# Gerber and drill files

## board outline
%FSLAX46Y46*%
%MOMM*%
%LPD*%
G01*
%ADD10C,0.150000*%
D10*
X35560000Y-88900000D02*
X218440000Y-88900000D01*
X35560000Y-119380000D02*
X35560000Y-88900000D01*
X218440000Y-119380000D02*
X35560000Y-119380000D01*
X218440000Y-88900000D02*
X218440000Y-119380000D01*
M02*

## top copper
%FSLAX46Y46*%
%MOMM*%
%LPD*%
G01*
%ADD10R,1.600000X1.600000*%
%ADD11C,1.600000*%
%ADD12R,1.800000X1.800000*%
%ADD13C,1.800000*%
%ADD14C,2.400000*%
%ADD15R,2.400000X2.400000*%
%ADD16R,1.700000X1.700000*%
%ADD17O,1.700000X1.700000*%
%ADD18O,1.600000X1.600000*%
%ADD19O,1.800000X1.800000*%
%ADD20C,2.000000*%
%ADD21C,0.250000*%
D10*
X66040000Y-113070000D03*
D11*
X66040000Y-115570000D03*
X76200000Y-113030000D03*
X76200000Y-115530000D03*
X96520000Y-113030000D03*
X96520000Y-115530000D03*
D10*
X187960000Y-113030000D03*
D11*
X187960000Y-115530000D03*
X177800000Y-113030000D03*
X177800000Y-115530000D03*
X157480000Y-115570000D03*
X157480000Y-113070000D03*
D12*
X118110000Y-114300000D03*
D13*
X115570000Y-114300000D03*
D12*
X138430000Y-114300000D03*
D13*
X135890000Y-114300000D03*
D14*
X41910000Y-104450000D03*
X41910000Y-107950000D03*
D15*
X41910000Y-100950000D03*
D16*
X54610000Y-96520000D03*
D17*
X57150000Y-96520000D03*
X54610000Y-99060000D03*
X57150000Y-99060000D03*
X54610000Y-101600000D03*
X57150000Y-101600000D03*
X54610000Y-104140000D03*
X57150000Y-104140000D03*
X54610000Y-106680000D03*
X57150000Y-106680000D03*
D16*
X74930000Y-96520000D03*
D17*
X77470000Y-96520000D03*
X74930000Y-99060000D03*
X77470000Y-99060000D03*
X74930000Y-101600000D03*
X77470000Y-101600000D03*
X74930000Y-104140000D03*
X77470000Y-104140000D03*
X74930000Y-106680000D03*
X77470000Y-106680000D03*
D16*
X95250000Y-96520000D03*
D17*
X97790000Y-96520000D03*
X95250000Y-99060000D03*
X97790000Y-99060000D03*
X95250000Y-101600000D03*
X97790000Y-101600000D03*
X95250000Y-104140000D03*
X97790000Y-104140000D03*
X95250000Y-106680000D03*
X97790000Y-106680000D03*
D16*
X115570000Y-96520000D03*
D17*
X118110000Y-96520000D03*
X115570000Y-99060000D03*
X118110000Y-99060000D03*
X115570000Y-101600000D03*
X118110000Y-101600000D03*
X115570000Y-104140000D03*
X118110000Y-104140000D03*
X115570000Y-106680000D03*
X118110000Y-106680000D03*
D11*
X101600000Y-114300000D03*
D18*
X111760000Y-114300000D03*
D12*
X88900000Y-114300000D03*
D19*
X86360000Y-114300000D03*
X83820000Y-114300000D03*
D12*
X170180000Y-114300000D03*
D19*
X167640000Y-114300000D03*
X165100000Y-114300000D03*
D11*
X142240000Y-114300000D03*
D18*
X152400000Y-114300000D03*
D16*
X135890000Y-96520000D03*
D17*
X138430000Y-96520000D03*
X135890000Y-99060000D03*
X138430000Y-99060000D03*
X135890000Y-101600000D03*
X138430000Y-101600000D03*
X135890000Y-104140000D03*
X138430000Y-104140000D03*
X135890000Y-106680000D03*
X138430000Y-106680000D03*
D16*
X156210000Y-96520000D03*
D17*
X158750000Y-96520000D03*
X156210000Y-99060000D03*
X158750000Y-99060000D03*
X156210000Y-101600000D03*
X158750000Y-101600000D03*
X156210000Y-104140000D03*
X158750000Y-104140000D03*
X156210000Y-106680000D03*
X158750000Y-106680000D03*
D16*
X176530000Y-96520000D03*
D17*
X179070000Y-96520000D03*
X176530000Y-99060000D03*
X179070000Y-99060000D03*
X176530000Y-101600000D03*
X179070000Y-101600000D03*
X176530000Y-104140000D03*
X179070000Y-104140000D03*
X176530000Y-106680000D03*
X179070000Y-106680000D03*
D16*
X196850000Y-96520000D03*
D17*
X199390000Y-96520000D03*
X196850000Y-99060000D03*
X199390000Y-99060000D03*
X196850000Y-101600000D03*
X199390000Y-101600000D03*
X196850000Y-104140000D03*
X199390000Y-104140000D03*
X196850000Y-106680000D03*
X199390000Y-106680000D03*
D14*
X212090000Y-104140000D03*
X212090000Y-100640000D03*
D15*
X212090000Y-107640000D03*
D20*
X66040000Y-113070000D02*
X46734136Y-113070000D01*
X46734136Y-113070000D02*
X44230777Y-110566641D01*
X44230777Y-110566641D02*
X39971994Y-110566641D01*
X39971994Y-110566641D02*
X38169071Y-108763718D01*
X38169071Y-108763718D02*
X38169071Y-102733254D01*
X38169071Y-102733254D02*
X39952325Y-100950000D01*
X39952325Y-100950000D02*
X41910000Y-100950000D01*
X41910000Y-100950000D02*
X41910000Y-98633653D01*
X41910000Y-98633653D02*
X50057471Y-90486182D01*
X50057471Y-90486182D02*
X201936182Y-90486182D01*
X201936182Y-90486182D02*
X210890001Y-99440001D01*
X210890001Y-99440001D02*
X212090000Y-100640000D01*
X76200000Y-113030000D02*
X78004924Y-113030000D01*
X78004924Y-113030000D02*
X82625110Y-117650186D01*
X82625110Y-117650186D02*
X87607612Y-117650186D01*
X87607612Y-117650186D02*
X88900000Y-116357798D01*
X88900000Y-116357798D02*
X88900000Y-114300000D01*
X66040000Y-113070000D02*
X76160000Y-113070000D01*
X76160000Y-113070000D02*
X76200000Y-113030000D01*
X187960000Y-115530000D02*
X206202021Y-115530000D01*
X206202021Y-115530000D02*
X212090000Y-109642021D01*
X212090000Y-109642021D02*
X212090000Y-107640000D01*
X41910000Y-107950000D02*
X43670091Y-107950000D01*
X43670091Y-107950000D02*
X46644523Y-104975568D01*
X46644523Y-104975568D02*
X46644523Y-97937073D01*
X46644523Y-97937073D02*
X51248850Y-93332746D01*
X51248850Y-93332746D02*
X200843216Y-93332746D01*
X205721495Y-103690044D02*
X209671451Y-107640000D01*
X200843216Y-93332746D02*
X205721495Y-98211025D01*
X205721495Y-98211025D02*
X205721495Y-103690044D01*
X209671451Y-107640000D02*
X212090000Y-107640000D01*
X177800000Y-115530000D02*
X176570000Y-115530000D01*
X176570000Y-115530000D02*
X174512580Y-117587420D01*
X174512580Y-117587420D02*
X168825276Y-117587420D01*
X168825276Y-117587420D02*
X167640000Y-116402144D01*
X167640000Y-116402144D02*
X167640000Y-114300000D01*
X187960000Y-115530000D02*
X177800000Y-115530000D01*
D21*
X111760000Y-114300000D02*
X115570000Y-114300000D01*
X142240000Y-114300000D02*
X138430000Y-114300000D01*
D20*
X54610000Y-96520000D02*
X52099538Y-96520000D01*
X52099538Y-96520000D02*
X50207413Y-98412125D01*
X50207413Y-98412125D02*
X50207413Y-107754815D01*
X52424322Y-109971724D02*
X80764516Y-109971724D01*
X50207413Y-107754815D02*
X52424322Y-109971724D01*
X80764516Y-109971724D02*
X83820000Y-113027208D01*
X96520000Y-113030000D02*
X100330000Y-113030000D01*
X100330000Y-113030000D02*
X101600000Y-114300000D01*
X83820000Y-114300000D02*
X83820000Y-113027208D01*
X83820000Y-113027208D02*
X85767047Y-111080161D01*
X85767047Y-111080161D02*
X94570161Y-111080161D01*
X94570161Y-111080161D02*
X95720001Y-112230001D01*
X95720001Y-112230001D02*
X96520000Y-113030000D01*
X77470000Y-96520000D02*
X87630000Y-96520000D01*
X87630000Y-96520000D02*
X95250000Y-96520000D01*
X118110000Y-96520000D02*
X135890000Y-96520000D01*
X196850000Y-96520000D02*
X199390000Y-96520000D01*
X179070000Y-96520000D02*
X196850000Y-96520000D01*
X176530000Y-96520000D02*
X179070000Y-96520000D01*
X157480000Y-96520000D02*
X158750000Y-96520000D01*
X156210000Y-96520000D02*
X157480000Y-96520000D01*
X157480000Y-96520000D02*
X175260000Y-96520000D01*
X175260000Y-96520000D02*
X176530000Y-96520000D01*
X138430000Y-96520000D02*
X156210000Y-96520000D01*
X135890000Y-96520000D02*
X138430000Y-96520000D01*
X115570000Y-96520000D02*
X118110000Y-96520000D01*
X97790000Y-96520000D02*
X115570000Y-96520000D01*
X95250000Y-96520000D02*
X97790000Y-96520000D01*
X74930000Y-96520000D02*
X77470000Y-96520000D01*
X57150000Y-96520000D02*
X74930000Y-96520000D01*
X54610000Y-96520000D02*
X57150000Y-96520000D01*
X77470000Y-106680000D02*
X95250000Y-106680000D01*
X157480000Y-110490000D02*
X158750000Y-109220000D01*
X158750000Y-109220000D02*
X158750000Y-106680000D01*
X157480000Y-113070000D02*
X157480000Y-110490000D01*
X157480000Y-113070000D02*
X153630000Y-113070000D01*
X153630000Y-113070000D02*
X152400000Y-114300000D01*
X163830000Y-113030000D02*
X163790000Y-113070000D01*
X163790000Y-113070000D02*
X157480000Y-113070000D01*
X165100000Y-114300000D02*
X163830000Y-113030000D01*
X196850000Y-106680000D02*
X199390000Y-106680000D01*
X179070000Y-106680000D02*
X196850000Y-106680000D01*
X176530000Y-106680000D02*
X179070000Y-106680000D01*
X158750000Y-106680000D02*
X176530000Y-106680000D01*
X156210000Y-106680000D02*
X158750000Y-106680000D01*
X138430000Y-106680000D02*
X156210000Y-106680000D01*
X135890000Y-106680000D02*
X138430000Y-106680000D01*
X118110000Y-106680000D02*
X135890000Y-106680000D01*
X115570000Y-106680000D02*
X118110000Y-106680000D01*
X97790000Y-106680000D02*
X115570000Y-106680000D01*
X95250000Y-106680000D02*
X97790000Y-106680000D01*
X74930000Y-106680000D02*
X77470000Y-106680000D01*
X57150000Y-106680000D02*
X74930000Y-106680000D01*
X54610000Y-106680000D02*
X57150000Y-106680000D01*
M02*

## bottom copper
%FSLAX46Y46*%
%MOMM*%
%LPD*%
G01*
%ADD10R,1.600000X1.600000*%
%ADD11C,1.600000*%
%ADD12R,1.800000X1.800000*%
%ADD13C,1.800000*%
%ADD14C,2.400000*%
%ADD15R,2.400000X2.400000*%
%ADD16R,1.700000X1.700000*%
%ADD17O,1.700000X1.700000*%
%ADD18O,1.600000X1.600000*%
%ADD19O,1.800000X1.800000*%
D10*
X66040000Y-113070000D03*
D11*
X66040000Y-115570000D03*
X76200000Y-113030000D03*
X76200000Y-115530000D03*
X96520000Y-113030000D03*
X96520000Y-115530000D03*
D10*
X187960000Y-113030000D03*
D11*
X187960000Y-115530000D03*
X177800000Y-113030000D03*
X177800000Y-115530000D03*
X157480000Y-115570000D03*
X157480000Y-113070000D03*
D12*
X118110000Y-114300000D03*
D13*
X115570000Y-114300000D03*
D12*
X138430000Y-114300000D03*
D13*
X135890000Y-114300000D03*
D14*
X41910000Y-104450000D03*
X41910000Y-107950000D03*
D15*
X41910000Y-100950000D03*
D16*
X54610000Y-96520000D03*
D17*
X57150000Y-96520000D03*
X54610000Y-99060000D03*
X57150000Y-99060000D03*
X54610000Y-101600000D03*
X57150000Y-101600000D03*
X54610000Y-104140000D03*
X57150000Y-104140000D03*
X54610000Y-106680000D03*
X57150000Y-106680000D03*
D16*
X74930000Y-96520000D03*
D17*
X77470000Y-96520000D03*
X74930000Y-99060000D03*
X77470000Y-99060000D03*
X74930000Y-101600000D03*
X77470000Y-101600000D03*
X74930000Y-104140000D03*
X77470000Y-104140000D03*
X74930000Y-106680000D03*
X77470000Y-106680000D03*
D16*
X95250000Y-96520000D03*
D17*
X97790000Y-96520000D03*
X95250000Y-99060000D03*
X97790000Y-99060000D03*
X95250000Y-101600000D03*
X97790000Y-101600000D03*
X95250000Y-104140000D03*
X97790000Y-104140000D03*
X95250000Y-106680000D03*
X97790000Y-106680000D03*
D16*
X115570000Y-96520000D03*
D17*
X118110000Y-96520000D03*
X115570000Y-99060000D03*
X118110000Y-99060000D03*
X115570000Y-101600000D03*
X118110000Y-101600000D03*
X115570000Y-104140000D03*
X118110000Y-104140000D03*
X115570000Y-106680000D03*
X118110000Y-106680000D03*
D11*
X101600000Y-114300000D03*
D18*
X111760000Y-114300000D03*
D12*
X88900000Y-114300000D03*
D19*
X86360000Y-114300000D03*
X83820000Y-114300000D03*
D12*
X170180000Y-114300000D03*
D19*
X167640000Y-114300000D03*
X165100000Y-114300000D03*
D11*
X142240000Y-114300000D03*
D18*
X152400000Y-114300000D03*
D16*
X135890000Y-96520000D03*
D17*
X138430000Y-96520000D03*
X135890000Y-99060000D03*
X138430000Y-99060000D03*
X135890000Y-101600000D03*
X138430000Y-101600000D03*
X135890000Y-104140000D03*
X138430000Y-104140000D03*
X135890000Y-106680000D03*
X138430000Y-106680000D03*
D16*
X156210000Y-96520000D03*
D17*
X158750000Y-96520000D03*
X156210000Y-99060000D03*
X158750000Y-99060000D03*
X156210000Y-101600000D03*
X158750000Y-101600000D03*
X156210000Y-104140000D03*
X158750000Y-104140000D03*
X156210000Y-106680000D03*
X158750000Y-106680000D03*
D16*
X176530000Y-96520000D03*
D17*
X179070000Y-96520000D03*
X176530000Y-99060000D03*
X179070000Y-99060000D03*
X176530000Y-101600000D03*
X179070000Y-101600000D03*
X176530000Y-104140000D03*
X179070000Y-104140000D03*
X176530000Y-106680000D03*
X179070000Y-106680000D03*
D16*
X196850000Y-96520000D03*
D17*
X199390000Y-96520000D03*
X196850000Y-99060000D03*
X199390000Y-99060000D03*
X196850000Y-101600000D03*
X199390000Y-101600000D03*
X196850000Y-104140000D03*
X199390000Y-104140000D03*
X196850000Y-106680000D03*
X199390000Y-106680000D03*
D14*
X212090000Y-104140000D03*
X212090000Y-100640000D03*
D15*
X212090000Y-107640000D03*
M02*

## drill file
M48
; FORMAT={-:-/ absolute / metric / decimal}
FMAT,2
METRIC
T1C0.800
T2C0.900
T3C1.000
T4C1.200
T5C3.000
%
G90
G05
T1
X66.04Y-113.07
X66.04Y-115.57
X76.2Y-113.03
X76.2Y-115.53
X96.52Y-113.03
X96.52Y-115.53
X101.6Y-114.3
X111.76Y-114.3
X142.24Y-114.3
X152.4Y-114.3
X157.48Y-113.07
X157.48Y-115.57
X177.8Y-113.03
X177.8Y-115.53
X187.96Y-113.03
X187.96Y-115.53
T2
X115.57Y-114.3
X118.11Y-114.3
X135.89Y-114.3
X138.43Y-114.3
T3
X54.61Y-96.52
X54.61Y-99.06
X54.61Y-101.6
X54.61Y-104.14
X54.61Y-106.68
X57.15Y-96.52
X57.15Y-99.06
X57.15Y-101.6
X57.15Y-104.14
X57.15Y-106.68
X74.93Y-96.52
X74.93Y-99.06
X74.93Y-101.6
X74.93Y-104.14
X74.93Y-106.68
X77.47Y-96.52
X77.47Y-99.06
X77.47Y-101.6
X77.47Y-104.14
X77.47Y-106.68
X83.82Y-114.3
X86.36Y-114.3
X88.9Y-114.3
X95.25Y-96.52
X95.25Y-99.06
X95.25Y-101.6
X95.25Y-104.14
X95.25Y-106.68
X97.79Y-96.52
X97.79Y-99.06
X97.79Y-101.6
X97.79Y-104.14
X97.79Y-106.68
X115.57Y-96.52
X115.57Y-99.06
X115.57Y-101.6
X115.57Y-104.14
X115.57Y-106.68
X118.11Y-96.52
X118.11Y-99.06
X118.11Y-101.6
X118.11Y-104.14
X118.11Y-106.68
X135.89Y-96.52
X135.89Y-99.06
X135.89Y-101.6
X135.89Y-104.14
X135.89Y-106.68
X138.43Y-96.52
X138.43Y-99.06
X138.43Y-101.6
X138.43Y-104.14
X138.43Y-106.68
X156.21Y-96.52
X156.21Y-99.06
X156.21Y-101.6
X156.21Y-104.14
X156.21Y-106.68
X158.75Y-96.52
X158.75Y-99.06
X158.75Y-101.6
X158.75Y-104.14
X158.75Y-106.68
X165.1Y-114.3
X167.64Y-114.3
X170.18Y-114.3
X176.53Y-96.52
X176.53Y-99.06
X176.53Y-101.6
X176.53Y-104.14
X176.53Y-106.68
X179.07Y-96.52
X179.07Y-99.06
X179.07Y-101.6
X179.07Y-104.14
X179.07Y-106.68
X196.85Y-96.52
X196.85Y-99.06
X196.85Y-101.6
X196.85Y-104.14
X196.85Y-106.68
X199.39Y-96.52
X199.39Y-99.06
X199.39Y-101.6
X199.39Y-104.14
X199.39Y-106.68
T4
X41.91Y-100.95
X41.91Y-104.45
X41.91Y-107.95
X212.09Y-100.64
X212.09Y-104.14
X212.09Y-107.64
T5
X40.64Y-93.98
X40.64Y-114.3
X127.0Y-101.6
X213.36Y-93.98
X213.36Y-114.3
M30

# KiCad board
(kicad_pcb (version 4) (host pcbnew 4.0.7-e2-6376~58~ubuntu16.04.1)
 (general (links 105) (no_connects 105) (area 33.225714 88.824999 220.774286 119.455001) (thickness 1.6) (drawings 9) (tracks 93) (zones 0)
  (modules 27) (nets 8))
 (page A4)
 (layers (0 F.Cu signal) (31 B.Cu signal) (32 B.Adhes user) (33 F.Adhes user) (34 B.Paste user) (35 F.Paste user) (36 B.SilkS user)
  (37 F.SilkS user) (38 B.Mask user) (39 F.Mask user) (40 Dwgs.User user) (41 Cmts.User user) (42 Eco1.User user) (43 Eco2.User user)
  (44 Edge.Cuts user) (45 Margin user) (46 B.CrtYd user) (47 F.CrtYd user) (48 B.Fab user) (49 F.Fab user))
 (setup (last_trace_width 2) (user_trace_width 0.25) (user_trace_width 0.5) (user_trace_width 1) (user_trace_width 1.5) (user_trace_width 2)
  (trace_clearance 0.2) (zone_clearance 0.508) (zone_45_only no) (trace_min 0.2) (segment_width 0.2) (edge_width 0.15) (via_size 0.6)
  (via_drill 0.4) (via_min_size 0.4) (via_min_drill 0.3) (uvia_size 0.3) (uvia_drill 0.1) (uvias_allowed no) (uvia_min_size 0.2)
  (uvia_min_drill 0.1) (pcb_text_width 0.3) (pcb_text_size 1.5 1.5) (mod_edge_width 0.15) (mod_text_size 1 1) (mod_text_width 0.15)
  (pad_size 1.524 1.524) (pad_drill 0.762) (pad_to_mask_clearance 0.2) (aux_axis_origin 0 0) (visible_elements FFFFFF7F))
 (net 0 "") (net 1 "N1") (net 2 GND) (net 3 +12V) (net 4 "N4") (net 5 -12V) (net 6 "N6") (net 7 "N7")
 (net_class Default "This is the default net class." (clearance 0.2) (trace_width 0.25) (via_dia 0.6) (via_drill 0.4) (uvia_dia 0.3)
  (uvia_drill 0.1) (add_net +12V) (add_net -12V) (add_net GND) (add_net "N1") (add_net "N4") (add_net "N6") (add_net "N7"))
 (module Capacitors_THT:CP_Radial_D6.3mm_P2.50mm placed (layer F.Cu) (at 66.04 113.07 270)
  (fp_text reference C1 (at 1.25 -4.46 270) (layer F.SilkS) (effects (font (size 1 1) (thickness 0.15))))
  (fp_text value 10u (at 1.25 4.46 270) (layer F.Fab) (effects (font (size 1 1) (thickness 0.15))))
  (pad 1 thru_hole rect (at 0 0 270) (size 1.6 1.6) (drill 0.8) (layers *.Cu *.Mask) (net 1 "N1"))
  (pad 2 thru_hole circle (at 2.5 0 270) (size 1.6 1.6) (drill 0.8) (layers *.Cu *.Mask) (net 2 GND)))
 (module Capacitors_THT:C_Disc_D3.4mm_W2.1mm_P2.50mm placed (layer F.Cu) (at 76.2 113.03 270)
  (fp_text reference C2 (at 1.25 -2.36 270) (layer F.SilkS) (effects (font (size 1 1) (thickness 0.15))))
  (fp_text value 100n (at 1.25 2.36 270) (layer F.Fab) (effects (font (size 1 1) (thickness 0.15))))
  (pad 1 thru_hole circle (at 0 0 270) (size 1.6 1.6) (drill 0.8) (layers *.Cu *.Mask) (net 1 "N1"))
  (pad 2 thru_hole circle (at 2.5 0 270) (size 1.6 1.6) (drill 0.8) (layers *.Cu *.Mask) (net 2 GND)))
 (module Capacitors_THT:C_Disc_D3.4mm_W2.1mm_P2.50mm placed (layer F.Cu) (at 96.52 113.03 270)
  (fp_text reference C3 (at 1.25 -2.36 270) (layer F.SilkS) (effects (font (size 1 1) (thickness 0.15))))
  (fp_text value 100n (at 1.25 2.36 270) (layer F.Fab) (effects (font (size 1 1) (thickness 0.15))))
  (pad 1 thru_hole circle (at 0 0 270) (size 1.6 1.6) (drill 0.8) (layers *.Cu *.Mask) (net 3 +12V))
  (pad 2 thru_hole circle (at 2.5 0 270) (size 1.6 1.6) (drill 0.8) (layers *.Cu *.Mask) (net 2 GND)))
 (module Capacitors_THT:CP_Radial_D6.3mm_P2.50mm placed (layer F.Cu) (at 187.96 113.03 270)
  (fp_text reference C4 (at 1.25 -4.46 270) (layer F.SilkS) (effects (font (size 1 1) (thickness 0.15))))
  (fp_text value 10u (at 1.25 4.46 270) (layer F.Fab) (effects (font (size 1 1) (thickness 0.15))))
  (pad 1 thru_hole rect (at 0 0 270) (size 1.6 1.6) (drill 0.8) (layers *.Cu *.Mask) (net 2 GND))
  (pad 2 thru_hole circle (at 2.5 0 270) (size 1.6 1.6) (drill 0.8) (layers *.Cu *.Mask) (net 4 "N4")))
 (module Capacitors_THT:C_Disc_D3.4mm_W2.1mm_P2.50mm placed (layer F.Cu) (at 177.8 113.03 270)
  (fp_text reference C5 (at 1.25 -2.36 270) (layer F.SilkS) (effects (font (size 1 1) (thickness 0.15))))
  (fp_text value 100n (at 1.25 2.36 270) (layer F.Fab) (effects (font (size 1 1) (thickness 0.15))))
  (pad 1 thru_hole circle (at 0 0 270) (size 1.6 1.6) (drill 0.8) (layers *.Cu *.Mask) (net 2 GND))
  (pad 2 thru_hole circle (at 2.5 0 270) (size 1.6 1.6) (drill 0.8) (layers *.Cu *.Mask) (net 4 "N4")))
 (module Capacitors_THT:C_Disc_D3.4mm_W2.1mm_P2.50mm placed (layer F.Cu) (at 157.48 115.57 90)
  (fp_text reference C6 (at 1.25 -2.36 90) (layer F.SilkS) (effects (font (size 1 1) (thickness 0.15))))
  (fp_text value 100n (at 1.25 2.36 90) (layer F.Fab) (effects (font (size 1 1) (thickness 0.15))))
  (pad 1 thru_hole circle (at 0 0 90) (size 1.6 1.6) (drill 0.8) (layers *.Cu *.Mask) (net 2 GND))
  (pad 2 thru_hole circle (at 2.5 0 90) (size 1.6 1.6) (drill 0.8) (layers *.Cu *.Mask) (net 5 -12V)))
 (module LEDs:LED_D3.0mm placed (layer F.Cu) (at 118.11 114.3 180)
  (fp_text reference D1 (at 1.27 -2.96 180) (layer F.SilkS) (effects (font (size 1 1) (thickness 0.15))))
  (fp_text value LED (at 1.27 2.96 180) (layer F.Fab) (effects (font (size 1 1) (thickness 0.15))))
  (pad 1 thru_hole rect (at 0 0 180) (size 1.8 1.8) (drill 0.9) (layers *.Cu *.Mask) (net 2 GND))
  (pad 2 thru_hole circle (at 2.54 0 180) (size 1.8 1.8) (drill 0.9) (layers *.Cu *.Mask) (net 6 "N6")))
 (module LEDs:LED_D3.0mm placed (layer F.Cu) (at 138.43 114.3 180)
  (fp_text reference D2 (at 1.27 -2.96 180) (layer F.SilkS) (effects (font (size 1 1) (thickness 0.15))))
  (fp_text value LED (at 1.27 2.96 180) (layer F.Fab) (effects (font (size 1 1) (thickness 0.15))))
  (pad 1 thru_hole rect (at 0 0 180) (size 1.8 1.8) (drill 0.9) (layers *.Cu *.Mask) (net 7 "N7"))
  (pad 2 thru_hole circle (at 2.54 0 180) (size 1.8 1.8) (drill 0.9) (layers *.Cu *.Mask) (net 2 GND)))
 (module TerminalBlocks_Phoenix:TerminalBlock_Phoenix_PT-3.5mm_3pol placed (layer F.Cu) (at 41.91 100.95 270)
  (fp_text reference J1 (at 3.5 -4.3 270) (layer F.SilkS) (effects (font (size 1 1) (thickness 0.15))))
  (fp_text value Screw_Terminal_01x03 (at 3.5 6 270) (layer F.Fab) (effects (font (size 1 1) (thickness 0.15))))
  (pad 2 thru_hole circle (at 3.5 0 270) (size 2.4 2.4) (drill 1.2) (layers *.Cu *.Mask) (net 2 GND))
  (pad 3 thru_hole circle (at 7 0 270) (size 2.4 2.4) (drill 1.2) (layers *.Cu *.Mask) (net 4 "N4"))
  (pad 1 thru_hole rect (at 0 0 270) (size 2.4 2.4) (drill 1.2) (layers *.Cu *.Mask) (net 1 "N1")))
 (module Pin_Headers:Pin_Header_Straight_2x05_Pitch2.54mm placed (layer F.Cu) (at 54.61 96.52)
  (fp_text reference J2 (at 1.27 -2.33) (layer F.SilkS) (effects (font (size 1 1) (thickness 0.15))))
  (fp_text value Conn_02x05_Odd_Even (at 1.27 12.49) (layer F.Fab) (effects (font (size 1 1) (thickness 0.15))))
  (pad 1 thru_hole rect (at 0 0) (size 1.7 1.7) (drill 1) (layers *.Cu *.Mask) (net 3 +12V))
  (pad 2 thru_hole oval (at 2.54 0) (size 1.7 1.7) (drill 1) (layers *.Cu *.Mask) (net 3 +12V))
  (pad 3 thru_hole oval (at 0 2.54) (size 1.7 1.7) (drill 1) (layers *.Cu *.Mask) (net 2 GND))
  (pad 4 thru_hole oval (at 2.54 2.54) (size 1.7 1.7) (drill 1) (layers *.Cu *.Mask) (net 2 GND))
  (pad 5 thru_hole oval (at 0 5.08) (size 1.7 1.7) (drill 1) (layers *.Cu *.Mask) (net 2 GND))
  (pad 6 thru_hole oval (at 2.54 5.08) (size 1.7 1.7) (drill 1) (layers *.Cu *.Mask) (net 2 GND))
  (pad 7 thru_hole oval (at 0 7.62) (size 1.7 1.7) (drill 1) (layers *.Cu *.Mask) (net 2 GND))
  (pad 8 thru_hole oval (at 2.54 7.62) (size 1.7 1.7) (drill 1) (layers *.Cu *.Mask) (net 2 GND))
  (pad 9 thru_hole oval (at 0 10.16) (size 1.7 1.7) (drill 1) (layers *.Cu *.Mask) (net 5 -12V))
  (pad 10 thru_hole oval (at 2.54 10.16) (size 1.7 1.7) (drill 1) (layers *.Cu *.Mask) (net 5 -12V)))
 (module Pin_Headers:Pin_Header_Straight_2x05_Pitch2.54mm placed (layer F.Cu) (at 74.93 96.52)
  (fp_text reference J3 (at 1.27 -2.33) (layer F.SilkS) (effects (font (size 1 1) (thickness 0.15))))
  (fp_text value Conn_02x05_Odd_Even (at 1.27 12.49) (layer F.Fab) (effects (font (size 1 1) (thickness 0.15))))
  (pad 1 thru_hole rect (at 0 0) (size 1.7 1.7) (drill 1) (layers *.Cu *.Mask) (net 3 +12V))
  (pad 2 thru_hole oval (at 2.54 0) (size 1.7 1.7) (drill 1) (layers *.Cu *.Mask) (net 3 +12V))
  (pad 3 thru_hole oval (at 0 2.54) (size 1.7 1.7) (drill 1) (layers *.Cu *.Mask) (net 2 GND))
  (pad 4 thru_hole oval (at 2.54 2.54) (size 1.7 1.7) (drill 1) (layers *.Cu *.Mask) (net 2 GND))
  (pad 5 thru_hole oval (at 0 5.08) (size 1.7 1.7) (drill 1) (layers *.Cu *.Mask) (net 2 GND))
  (pad 6 thru_hole oval (at 2.54 5.08) (size 1.7 1.7) (drill 1) (layers *.Cu *.Mask) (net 2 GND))
  (pad 7 thru_hole oval (at 0 7.62) (size 1.7 1.7) (drill 1) (layers *.Cu *.Mask) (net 2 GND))
  (pad 8 thru_hole oval (at 2.54 7.62) (size 1.7 1.7) (drill 1) (layers *.Cu *.Mask) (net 2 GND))
  (pad 9 thru_hole oval (at 0 10.16) (size 1.7 1.7) (drill 1) (layers *.Cu *.Mask) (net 5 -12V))
  (pad 10 thru_hole oval (at 2.54 10.16) (size 1.7 1.7) (drill 1) (layers *.Cu *.Mask) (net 5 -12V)))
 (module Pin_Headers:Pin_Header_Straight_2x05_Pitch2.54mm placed (layer F.Cu) (at 95.25 96.52)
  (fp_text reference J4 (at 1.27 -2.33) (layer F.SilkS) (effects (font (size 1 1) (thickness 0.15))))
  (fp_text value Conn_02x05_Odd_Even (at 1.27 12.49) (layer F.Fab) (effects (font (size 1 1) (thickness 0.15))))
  (pad 1 thru_hole rect (at 0 0) (size 1.7 1.7) (drill 1) (layers *.Cu *.Mask) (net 3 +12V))
  (pad 2 thru_hole oval (at 2.54 0) (size 1.7 1.7) (drill 1) (layers *.Cu *.Mask) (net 3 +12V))
  (pad 3 thru_hole oval (at 0 2.54) (size 1.7 1.7) (drill 1) (layers *.Cu *.Mask) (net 2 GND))
  (pad 4 thru_hole oval (at 2.54 2.54) (size 1.7 1.7) (drill 1) (layers *.Cu *.Mask) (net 2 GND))
  (pad 5 thru_hole oval (at 0 5.08) (size 1.7 1.7) (drill 1) (layers *.Cu *.Mask) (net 2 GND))
  (pad 6 thru_hole oval (at 2.54 5.08) (size 1.7 1.7) (drill 1) (layers *.Cu *.Mask) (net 2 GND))
  (pad 7 thru_hole oval (at 0 7.62) (size 1.7 1.7) (drill 1) (layers *.Cu *.Mask) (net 2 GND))
  (pad 8 thru_hole oval (at 2.54 7.62) (size 1.7 1.7) (drill 1) (layers *.Cu *.Mask) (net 2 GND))
  (pad 9 thru_hole oval (at 0 10.16) (size 1.7 1.7) (drill 1) (layers *.Cu *.Mask) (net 5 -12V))
  (pad 10 thru_hole oval (at 2.54 10.16) (size 1.7 1.7) (drill 1) (layers *.Cu *.Mask) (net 5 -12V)))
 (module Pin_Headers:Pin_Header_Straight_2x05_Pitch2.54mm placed (layer F.Cu) (at 115.57 96.52)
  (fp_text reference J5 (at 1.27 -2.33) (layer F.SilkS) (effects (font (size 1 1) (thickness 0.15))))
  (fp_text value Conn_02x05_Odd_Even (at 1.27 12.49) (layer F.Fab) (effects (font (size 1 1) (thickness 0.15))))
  (pad 1 thru_hole rect (at 0 0) (size 1.7 1.7) (drill 1) (layers *.Cu *.Mask) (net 3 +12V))
  (pad 2 thru_hole oval (at 2.54 0) (size 1.7 1.7) (drill 1) (layers *.Cu *.Mask) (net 3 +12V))
  (pad 3 thru_hole oval (at 0 2.54) (size 1.7 1.7) (drill 1) (layers *.Cu *.Mask) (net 2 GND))
  (pad 4 thru_hole oval (at 2.54 2.54) (size 1.7 1.7) (drill 1) (layers *.Cu *.Mask) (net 2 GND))
  (pad 5 thru_hole oval (at 0 5.08) (size 1.7 1.7) (drill 1) (layers *.Cu *.Mask) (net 2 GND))
  (pad 6 thru_hole oval (at 2.54 5.08) (size 1.7 1.7) (drill 1) (layers *.Cu *.Mask) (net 2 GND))
  (pad 7 thru_hole oval (at 0 7.62) (size 1.7 1.7) (drill 1) (layers *.Cu *.Mask) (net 2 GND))
  (pad 8 thru_hole oval (at 2.54 7.62) (size 1.7 1.7) (drill 1) (layers *.Cu *.Mask) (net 2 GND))
  (pad 9 thru_hole oval (at 0 10.16) (size 1.7 1.7) (drill 1) (layers *.Cu *.Mask) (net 5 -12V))
  (pad 10 thru_hole oval (at 2.54 10.16) (size 1.7 1.7) (drill 1) (layers *.Cu *.Mask) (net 5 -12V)))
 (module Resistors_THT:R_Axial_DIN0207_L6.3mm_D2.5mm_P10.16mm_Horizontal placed (layer F.Cu) (at 101.6 114.3)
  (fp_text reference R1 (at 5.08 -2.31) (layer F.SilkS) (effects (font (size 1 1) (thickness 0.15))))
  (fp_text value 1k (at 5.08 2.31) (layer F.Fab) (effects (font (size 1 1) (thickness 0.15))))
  (pad 1 thru_hole circle (at 0 0) (size 1.6 1.6) (drill 0.8) (layers *.Cu *.Mask) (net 3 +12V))
  (pad 2 thru_hole oval (at 10.16 0) (size 1.6 1.6) (drill 0.8) (layers *.Cu *.Mask) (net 6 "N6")))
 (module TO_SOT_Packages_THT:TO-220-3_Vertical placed (layer F.Cu) (at 88.9 114.3 180)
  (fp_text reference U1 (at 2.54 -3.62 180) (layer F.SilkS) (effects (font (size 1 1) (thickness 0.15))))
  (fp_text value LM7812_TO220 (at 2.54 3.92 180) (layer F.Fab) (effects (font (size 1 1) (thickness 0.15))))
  (pad 1 thru_hole rect (at 0 0 180) (size 1.8 1.8) (drill 1) (layers *.Cu *.Mask) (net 1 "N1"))
  (pad 2 thru_hole oval (at 2.54 0 180) (size 1.8 1.8) (drill 1) (layers *.Cu *.Mask) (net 2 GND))
  (pad 3 thru_hole oval (at 5.08 0 180) (size 1.8 1.8) (drill 1) (layers *.Cu *.Mask) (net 3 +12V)))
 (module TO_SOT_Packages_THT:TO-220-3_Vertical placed (layer F.Cu) (at 170.18 114.3 180)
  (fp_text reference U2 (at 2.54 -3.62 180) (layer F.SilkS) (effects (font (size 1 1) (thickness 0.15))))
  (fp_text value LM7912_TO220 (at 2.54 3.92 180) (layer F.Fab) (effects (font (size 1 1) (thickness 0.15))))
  (pad 1 thru_hole rect (at 0 0 180) (size 1.8 1.8) (drill 1) (layers *.Cu *.Mask) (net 2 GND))
  (pad 2 thru_hole oval (at 2.54 0 180) (size 1.8 1.8) (drill 1) (layers *.Cu *.Mask) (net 4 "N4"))
  (pad 3 thru_hole oval (at 5.08 0 180) (size 1.8 1.8) (drill 1) (layers *.Cu *.Mask) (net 5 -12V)))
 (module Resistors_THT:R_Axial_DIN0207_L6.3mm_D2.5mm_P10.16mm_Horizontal (layer F.Cu) (at 142.24 114.3)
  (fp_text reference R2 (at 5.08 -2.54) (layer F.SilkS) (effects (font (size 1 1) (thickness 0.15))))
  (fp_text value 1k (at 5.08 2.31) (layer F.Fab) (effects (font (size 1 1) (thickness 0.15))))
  (pad 1 thru_hole circle (at 0 0) (size 1.6 1.6) (drill 0.8) (layers *.Cu *.Mask) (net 7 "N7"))
  (pad 2 thru_hole oval (at 10.16 0) (size 1.6 1.6) (drill 0.8) (layers *.Cu *.Mask) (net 5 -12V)))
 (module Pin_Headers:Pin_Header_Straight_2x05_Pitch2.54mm (layer F.Cu) (at 135.89 96.52)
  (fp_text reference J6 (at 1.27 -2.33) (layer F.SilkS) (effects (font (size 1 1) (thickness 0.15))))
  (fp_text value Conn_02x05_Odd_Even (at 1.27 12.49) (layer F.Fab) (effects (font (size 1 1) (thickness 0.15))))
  (pad 1 thru_hole rect (at 0 0) (size 1.7 1.7) (drill 1) (layers *.Cu *.Mask) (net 3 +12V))
  (pad 2 thru_hole oval (at 2.54 0) (size 1.7 1.7) (drill 1) (layers *.Cu *.Mask) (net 3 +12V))
  (pad 3 thru_hole oval (at 0 2.54) (size 1.7 1.7) (drill 1) (layers *.Cu *.Mask) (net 2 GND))
  (pad 4 thru_hole oval (at 2.54 2.54) (size 1.7 1.7) (drill 1) (layers *.Cu *.Mask) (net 2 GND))
  (pad 5 thru_hole oval (at 0 5.08) (size 1.7 1.7) (drill 1) (layers *.Cu *.Mask) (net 2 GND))
  (pad 6 thru_hole oval (at 2.54 5.08) (size 1.7 1.7) (drill 1) (layers *.Cu *.Mask) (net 2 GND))
  (pad 7 thru_hole oval (at 0 7.62) (size 1.7 1.7) (drill 1) (layers *.Cu *.Mask) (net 2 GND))
  (pad 8 thru_hole oval (at 2.54 7.62) (size 1.7 1.7) (drill 1) (layers *.Cu *.Mask) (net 2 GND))
  (pad 9 thru_hole oval (at 0 10.16) (size 1.7 1.7) (drill 1) (layers *.Cu *.Mask) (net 5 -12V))
  (pad 10 thru_hole oval (at 2.54 10.16) (size 1.7 1.7) (drill 1) (layers *.Cu *.Mask) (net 5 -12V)))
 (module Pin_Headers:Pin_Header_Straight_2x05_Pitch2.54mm (layer F.Cu) (at 156.21 96.52)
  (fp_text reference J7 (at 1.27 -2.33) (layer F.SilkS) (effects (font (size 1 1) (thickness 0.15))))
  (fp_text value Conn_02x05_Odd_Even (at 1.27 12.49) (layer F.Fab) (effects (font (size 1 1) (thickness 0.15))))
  (pad 1 thru_hole rect (at 0 0) (size 1.7 1.7) (drill 1) (layers *.Cu *.Mask) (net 3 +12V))
  (pad 2 thru_hole oval (at 2.54 0) (size 1.7 1.7) (drill 1) (layers *.Cu *.Mask) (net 3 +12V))
  (pad 3 thru_hole oval (at 0 2.54) (size 1.7 1.7) (drill 1) (layers *.Cu *.Mask) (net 2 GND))
  (pad 4 thru_hole oval (at 2.54 2.54) (size 1.7 1.7) (drill 1) (layers *.Cu *.Mask) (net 2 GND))
  (pad 5 thru_hole oval (at 0 5.08) (size 1.7 1.7) (drill 1) (layers *.Cu *.Mask) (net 2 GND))
  (pad 6 thru_hole oval (at 2.54 5.08) (size 1.7 1.7) (drill 1) (layers *.Cu *.Mask) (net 2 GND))
  (pad 7 thru_hole oval (at 0 7.62) (size 1.7 1.7) (drill 1) (layers *.Cu *.Mask) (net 2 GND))
  (pad 8 thru_hole oval (at 2.54 7.62) (size 1.7 1.7) (drill 1) (layers *.Cu *.Mask) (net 2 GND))
  (pad 9 thru_hole oval (at 0 10.16) (size 1.7 1.7) (drill 1) (layers *.Cu *.Mask) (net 5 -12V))
  (pad 10 thru_hole oval (at 2.54 10.16) (size 1.7 1.7) (drill 1) (layers *.Cu *.Mask) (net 5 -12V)))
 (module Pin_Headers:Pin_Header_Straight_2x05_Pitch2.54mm (layer F.Cu) (at 176.53 96.52)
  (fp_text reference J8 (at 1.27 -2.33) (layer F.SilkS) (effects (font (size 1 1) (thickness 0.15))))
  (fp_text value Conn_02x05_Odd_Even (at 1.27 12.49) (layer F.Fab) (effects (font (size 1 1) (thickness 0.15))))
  (pad 1 thru_hole rect (at 0 0) (size 1.7 1.7) (drill 1) (layers *.Cu *.Mask) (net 3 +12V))
  (pad 2 thru_hole oval (at 2.54 0) (size 1.7 1.7) (drill 1) (layers *.Cu *.Mask) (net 3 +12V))
  (pad 3 thru_hole oval (at 0 2.54) (size 1.7 1.7) (drill 1) (layers *.Cu *.Mask) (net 2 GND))
  (pad 4 thru_hole oval (at 2.54 2.54) (size 1.7 1.7) (drill 1) (layers *.Cu *.Mask) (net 2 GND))
  (pad 5 thru_hole oval (at 0 5.08) (size 1.7 1.7) (drill 1) (layers *.Cu *.Mask) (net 2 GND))
  (pad 6 thru_hole oval (at 2.54 5.08) (size 1.7 1.7) (drill 1) (layers *.Cu *.Mask) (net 2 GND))
  (pad 7 thru_hole oval (at 0 7.62) (size 1.7 1.7) (drill 1) (layers *.Cu *.Mask) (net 2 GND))
  (pad 8 thru_hole oval (at 2.54 7.62) (size 1.7 1.7) (drill 1) (layers *.Cu *.Mask) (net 2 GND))
  (pad 9 thru_hole oval (at 0 10.16) (size 1.7 1.7) (drill 1) (layers *.Cu *.Mask) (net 5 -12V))
  (pad 10 thru_hole oval (at 2.54 10.16) (size 1.7 1.7) (drill 1) (layers *.Cu *.Mask) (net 5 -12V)))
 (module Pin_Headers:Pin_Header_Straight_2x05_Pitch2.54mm (layer F.Cu) (at 196.85 96.52)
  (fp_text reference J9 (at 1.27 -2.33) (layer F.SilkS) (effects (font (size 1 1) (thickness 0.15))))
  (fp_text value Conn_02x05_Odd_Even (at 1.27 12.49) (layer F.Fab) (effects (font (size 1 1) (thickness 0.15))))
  (pad 1 thru_hole rect (at 0 0) (size 1.7 1.7) (drill 1) (layers *.Cu *.Mask) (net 3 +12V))
  (pad 2 thru_hole oval (at 2.54 0) (size 1.7 1.7) (drill 1) (layers *.Cu *.Mask) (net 3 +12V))
  (pad 3 thru_hole oval (at 0 2.54) (size 1.7 1.7) (drill 1) (layers *.Cu *.Mask) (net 2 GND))
  (pad 4 thru_hole oval (at 2.54 2.54) (size 1.7 1.7) (drill 1) (layers *.Cu *.Mask) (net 2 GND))
  (pad 5 thru_hole oval (at 0 5.08) (size 1.7 1.7) (drill 1) (layers *.Cu *.Mask) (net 2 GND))
  (pad 6 thru_hole oval (at 2.54 5.08) (size 1.7 1.7) (drill 1) (layers *.Cu *.Mask) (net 2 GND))
  (pad 7 thru_hole oval (at 0 7.62) (size 1.7 1.7) (drill 1) (layers *.Cu *.Mask) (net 2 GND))
  (pad 8 thru_hole oval (at 2.54 7.62) (size 1.7 1.7) (drill 1) (layers *.Cu *.Mask) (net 2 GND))
  (pad 9 thru_hole oval (at 0 10.16) (size 1.7 1.7) (drill 1) (layers *.Cu *.Mask) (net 5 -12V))
  (pad 10 thru_hole oval (at 2.54 10.16) (size 1.7 1.7) (drill 1) (layers *.Cu *.Mask) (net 5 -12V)))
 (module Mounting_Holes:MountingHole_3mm (layer F.Cu) (at 40.64 93.98)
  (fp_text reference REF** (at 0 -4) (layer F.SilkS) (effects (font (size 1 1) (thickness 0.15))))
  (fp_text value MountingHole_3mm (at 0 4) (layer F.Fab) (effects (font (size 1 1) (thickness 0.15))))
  (pad 1 np_thru_hole circle (at 0 0) (size 3 3) (drill 3) (layers *.Cu *.Mask)))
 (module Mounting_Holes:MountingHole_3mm (layer F.Cu) (at 213.36 114.3)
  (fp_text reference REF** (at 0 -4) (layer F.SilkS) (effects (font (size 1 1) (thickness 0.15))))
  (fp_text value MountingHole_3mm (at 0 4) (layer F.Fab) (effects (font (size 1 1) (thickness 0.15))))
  (pad 1 np_thru_hole circle (at 0 0) (size 3 3) (drill 3) (layers *.Cu *.Mask)))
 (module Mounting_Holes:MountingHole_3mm (layer F.Cu) (at 213.36 93.98)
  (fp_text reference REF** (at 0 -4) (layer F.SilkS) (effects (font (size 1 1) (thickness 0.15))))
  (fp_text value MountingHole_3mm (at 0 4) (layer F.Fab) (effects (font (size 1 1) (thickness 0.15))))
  (pad 1 np_thru_hole circle (at 0 0) (size 3 3) (drill 3) (layers *.Cu *.Mask)))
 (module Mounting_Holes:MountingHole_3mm (layer F.Cu) (at 40.64 114.3)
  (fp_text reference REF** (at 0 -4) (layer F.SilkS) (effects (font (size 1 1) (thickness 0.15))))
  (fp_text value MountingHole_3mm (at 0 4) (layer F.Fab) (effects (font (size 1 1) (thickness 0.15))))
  (pad 1 np_thru_hole circle (at 0 0) (size 3 3) (drill 3) (layers *.Cu *.Mask)))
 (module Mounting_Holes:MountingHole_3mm (layer F.Cu) (at 127 101.6)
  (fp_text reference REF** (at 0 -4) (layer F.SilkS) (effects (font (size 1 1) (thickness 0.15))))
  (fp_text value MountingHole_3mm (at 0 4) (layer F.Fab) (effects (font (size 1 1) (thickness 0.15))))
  (pad 1 np_thru_hole circle (at 0 0) (size 3 3) (drill 3) (layers *.Cu *.Mask)))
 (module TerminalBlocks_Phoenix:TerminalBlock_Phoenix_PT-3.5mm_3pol (layer F.Cu) (at 212.09 107.64 90)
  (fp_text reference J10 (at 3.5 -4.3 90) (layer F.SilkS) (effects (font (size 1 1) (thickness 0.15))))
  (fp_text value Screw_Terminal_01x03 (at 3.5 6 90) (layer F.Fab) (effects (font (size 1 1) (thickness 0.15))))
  (pad 2 thru_hole circle (at 3.5 0 90) (size 2.4 2.4) (drill 1.2) (layers *.Cu *.Mask) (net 2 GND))
  (pad 3 thru_hole circle (at 7 0 90) (size 2.4 2.4) (drill 1.2) (layers *.Cu *.Mask) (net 1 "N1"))
  (pad 1 thru_hole rect (at 0 0 90) (size 2.4 2.4) (drill 1.2) (layers *.Cu *.Mask) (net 4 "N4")))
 (gr_line (start 35.56 88.9) (end 218.44 88.9) (layer Edge.Cuts) (width 0.15))
 (gr_line (start 35.56 119.38) (end 35.56 88.9) (layer Edge.Cuts) (width 0.15))
 (gr_line (start 218.44 119.38) (end 35.56 119.38) (layer Edge.Cuts) (width 0.15))
 (gr_line (start 218.44 88.9) (end 218.44 119.38) (layer Edge.Cuts) (width 0.15))
 (segment (start 66.04 113.07) (end 46.734136 113.07) (width 2) (layer F.Cu) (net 1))
 (segment (start 46.734136 113.07) (end 44.230777 110.566641) (width 2) (layer F.Cu) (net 1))
 (segment (start 44.230777 110.566641) (end 39.971994 110.566641) (width 2) (layer F.Cu) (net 1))
 (segment (start 39.971994 110.566641) (end 38.169071 108.763718) (width 2) (layer F.Cu) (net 1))
 (segment (start 38.169071 108.763718) (end 38.169071 102.733254) (width 2) (layer F.Cu) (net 1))
 (segment (start 38.169071 102.733254) (end 39.952325 100.95) (width 2) (layer F.Cu) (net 1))
 (segment (start 39.952325 100.95) (end 41.91 100.95) (width 2) (layer F.Cu) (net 1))
 (segment (start 41.91 100.95) (end 41.91 98.633653) (width 2) (layer F.Cu) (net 1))
 (segment (start 41.91 98.633653) (end 50.057471 90.486182) (width 2) (layer F.Cu) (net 1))
 (segment (start 50.057471 90.486182) (end 201.936182 90.486182) (width 2) (layer F.Cu) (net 1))
 (segment (start 201.936182 90.486182) (end 210.890001 99.440001) (width 2) (layer F.Cu) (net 1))
 (segment (start 210.890001 99.440001) (end 212.09 100.64) (width 2) (layer F.Cu) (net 1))
 (segment (start 76.2 113.03) (end 78.004924 113.03) (width 2) (layer F.Cu) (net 1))
 (segment (start 78.004924 113.03) (end 82.62511 117.650186) (width 2) (layer F.Cu) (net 1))
 (segment (start 82.62511 117.650186) (end 87.607612 117.650186) (width 2) (layer F.Cu) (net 1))
 (segment (start 87.607612 117.650186) (end 88.9 116.357798) (width 2) (layer F.Cu) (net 1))
 (segment (start 88.9 116.357798) (end 88.9 114.3) (width 2) (layer F.Cu) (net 1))
 (segment (start 66.04 113.07) (end 76.16 113.07) (width 2) (layer F.Cu) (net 1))
 (segment (start 76.16 113.07) (end 76.2 113.03) (width 2) (layer F.Cu) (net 1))
 (segment (start 187.96 115.53) (end 206.202021 115.53) (width 2) (layer F.Cu) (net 4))
 (segment (start 206.202021 115.53) (end 212.09 109.642021) (width 2) (layer F.Cu) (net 4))
 (segment (start 212.09 109.642021) (end 212.09 107.64) (width 2) (layer F.Cu) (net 4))
 (segment (start 41.91 107.95) (end 43.670091 107.95) (width 2) (layer F.Cu) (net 4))
 (segment (start 43.670091 107.95) (end 46.644523 104.975568) (width 2) (layer F.Cu) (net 4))
 (segment (start 46.644523 104.975568) (end 46.644523 97.937073) (width 2) (layer F.Cu) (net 4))
 (segment (start 46.644523 97.937073) (end 51.24885 93.332746) (width 2) (layer F.Cu) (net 4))
 (segment (start 51.24885 93.332746) (end 200.843216 93.332746) (width 2) (layer F.Cu) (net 4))
 (segment (start 205.721495 103.690044) (end 209.671451 107.64) (width 2) (layer F.Cu) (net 4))
 (segment (start 200.843216 93.332746) (end 205.721495 98.211025) (width 2) (layer F.Cu) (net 4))
 (segment (start 205.721495 98.211025) (end 205.721495 103.690044) (width 2) (layer F.Cu) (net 4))
 (segment (start 209.671451 107.64) (end 212.09 107.64) (width 2) (layer F.Cu) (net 4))
 (segment (start 177.8 115.53) (end 176.57 115.53) (width 2) (layer F.Cu) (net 4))
 (segment (start 176.57 115.53) (end 174.51258 117.58742) (width 2) (layer F.Cu) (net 4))
 (segment (start 174.51258 117.58742) (end 168.825276 117.58742) (width 2) (layer F.Cu) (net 4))
 (segment (start 168.825276 117.58742) (end 167.64 116.402144) (width 2) (layer F.Cu) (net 4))
 (segment (start 167.64 116.402144) (end 167.64 114.3) (width 2) (layer F.Cu) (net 4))
 (segment (start 187.96 115.53) (end 177.8 115.53) (width 2) (layer F.Cu) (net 4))
 (segment (start 111.76 114.3) (end 115.57 114.3) (width 0.25) (layer F.Cu) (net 6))
 (segment (start 142.24 114.3) (end 138.43 114.3) (width 0.25) (layer F.Cu) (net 7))
 (segment (start 54.61 96.52) (end 52.099538 96.52) (width 2) (layer F.Cu) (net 3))
 (segment (start 52.099538 96.52) (end 50.207413 98.412125) (width 2) (layer F.Cu) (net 3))
 (segment (start 50.207413 98.412125) (end 50.207413 107.754815) (width 2) (layer F.Cu) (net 3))
 (segment (start 52.424322 109.971724) (end 80.764516 109.971724) (width 2) (layer F.Cu) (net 3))
 (segment (start 50.207413 107.754815) (end 52.424322 109.971724) (width 2) (layer F.Cu) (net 3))
 (segment (start 80.764516 109.971724) (end 83.82 113.027208) (width 2) (layer F.Cu) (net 3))
 (segment (start 96.52 113.03) (end 100.33 113.03) (width 2) (layer F.Cu) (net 3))
 (segment (start 100.33 113.03) (end 101.6 114.3) (width 2) (layer F.Cu) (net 3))
 (segment (start 83.82 114.3) (end 83.82 113.027208) (width 2) (layer F.Cu) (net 3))
 (segment (start 83.82 113.027208) (end 85.767047 111.080161) (width 2) (layer F.Cu) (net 3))
 (segment (start 85.767047 111.080161) (end 94.570161 111.080161) (width 2) (layer F.Cu) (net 3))
 (segment (start 94.570161 111.080161) (end 95.720001 112.230001) (width 2) (layer F.Cu) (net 3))
 (segment (start 95.720001 112.230001) (end 96.52 113.03) (width 2) (layer F.Cu) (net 3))
 (segment (start 77.47 96.52) (end 87.63 96.52) (width 2) (layer F.Cu) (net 3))
 (segment (start 87.63 96.52) (end 95.25 96.52) (width 2) (layer F.Cu) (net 3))
 (segment (start 118.11 96.52) (end 135.89 96.52) (width 2) (layer F.Cu) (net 3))
 (segment (start 196.85 96.52) (end 199.39 96.52) (width 2) (layer F.Cu) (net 3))
 (segment (start 179.07 96.52) (end 196.85 96.52) (width 2) (layer F.Cu) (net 3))
 (segment (start 176.53 96.52) (end 179.07 96.52) (width 2) (layer F.Cu) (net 3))
 (segment (start 157.48 96.52) (end 158.75 96.52) (width 2) (layer F.Cu) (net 3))
 (segment (start 156.21 96.52) (end 157.48 96.52) (width 2) (layer F.Cu) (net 3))
 (segment (start 157.48 96.52) (end 175.26 96.52) (width 2) (layer F.Cu) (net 3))
 (segment (start 175.26 96.52) (end 176.53 96.52) (width 2) (layer F.Cu) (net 3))
 (segment (start 138.43 96.52) (end 156.21 96.52) (width 2) (layer F.Cu) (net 3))
 (segment (start 135.89 96.52) (end 138.43 96.52) (width 2) (layer F.Cu) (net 3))
 (segment (start 115.57 96.52) (end 118.11 96.52) (width 2) (layer F.Cu) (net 3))
 (segment (start 97.79 96.52) (end 115.57 96.52) (width 2) (layer F.Cu) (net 3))
 (segment (start 95.25 96.52) (end 97.79 96.52) (width 2) (layer F.Cu) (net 3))
 (segment (start 74.93 96.52) (end 77.47 96.52) (width 2) (layer F.Cu) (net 3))
 (segment (start 57.15 96.52) (end 74.93 96.52) (width 2) (layer F.Cu) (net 3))
 (segment (start 54.61 96.52) (end 57.15 96.52) (width 2) (layer F.Cu) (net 3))
 (segment (start 77.47 106.68) (end 95.25 106.68) (width 2) (layer F.Cu) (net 5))
 (segment (start 157.48 110.49) (end 158.75 109.22) (width 2) (layer F.Cu) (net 5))
 (segment (start 158.75 109.22) (end 158.75 106.68) (width 2) (layer F.Cu) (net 5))
 (segment (start 157.48 113.07) (end 157.48 110.49) (width 2) (layer F.Cu) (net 5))
 (segment (start 157.48 113.07) (end 153.63 113.07) (width 2) (layer F.Cu) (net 5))
 (segment (start 153.63 113.07) (end 152.4 114.3) (width 2) (layer F.Cu) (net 5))
 (segment (start 163.83 113.03) (end 163.79 113.07) (width 2) (layer F.Cu) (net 5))
 (segment (start 163.79 113.07) (end 157.48 113.07) (width 2) (layer F.Cu) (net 5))
 (segment (start 165.1 114.3) (end 163.83 113.03) (width 2) (layer F.Cu) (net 5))
 (segment (start 196.85 106.68) (end 199.39 106.68) (width 2) (layer F.Cu) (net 5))
 (segment (start 179.07 106.68) (end 196.85 106.68) (width 2) (layer F.Cu) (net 5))
 (segment (start 176.53 106.68) (end 179.07 106.68) (width 2) (layer F.Cu) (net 5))
 (segment (start 158.75 106.68) (end 176.53 106.68) (width 2) (layer F.Cu) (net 5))
 (segment (start 156.21 106.68) (end 158.75 106.68) (width 2) (layer F.Cu) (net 5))
 (segment (start 138.43 106.68) (end 156.21 106.68) (width 2) (layer F.Cu) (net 5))
 (segment (start 135.89 106.68) (end 138.43 106.68) (width 2) (layer F.Cu) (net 5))
 (segment (start 118.11 106.68) (end 135.89 106.68) (width 2) (layer F.Cu) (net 5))
 (segment (start 115.57 106.68) (end 118.11 106.68) (width 2) (layer F.Cu) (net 5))
 (segment (start 97.79 106.68) (end 115.57 106.68) (width 2) (layer F.Cu) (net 5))
 (segment (start 95.25 106.68) (end 97.79 106.68) (width 2) (layer F.Cu) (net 5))
 (segment (start 74.93 106.68) (end 77.47 106.68) (width 2) (layer F.Cu) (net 5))
 (segment (start 57.15 106.68) (end 74.93 106.68) (width 2) (layer F.Cu) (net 5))
 (segment (start 54.61 106.68) (end 57.15 106.68) (width 2) (layer F.Cu) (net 5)))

